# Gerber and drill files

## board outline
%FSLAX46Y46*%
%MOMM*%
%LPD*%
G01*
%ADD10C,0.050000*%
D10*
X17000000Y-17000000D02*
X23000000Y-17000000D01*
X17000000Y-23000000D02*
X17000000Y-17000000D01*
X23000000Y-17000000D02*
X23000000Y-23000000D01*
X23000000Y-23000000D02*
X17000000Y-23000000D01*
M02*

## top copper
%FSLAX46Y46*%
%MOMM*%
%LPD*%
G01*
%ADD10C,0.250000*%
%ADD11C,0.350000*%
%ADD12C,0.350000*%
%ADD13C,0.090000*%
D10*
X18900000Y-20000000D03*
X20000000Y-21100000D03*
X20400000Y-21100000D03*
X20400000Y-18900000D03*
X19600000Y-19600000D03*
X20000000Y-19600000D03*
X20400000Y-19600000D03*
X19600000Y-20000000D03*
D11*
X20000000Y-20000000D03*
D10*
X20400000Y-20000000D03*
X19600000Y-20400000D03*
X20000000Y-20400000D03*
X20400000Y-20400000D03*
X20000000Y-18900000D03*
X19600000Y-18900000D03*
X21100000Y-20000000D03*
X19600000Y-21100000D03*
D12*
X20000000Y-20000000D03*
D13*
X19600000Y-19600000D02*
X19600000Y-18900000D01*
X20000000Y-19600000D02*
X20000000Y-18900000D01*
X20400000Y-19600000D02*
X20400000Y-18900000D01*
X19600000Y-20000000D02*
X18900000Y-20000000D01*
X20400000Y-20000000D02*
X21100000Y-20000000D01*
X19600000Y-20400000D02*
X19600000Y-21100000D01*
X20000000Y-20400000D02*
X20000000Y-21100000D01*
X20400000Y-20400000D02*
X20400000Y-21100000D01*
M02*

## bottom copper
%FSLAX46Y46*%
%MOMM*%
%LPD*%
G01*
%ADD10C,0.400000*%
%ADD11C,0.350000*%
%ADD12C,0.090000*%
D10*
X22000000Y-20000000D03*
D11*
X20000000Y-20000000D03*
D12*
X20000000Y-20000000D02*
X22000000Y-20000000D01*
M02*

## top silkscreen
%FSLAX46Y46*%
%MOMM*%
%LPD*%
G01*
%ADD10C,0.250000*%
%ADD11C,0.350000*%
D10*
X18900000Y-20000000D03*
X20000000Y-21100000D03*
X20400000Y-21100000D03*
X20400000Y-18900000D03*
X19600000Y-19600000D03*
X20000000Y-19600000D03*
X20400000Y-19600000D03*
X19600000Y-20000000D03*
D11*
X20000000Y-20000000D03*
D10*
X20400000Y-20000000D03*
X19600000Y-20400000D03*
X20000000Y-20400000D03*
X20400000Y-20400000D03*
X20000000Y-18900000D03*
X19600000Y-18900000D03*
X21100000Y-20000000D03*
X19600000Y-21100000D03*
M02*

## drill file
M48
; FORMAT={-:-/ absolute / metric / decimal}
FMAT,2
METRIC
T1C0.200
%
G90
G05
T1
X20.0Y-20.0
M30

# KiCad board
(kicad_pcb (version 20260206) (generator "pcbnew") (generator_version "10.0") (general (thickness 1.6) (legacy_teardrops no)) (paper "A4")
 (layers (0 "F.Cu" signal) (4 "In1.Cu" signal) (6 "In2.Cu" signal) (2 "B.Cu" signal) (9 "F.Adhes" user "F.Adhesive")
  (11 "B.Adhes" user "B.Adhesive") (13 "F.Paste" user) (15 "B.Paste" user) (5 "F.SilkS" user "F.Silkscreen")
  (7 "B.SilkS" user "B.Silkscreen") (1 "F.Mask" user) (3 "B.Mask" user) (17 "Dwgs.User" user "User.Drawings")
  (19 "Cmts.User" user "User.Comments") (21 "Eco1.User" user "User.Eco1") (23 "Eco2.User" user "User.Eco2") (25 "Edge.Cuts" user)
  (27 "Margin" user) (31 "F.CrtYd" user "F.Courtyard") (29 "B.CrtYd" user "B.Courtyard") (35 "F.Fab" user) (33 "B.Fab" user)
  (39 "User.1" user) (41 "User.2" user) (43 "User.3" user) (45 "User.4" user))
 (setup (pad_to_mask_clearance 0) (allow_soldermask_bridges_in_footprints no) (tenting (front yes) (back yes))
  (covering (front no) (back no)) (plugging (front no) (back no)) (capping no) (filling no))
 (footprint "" (layer "F.Cu") (at 18.9 20)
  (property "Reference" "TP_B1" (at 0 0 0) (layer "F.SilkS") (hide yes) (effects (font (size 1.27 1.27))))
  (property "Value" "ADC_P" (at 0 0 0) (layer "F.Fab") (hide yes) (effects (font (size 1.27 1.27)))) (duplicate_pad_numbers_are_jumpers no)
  (pad "1" smd circle (at 0 0) (size 0.25 0.25) (layers "F.Cu" "F.Mask" "F.SilkS" "F.Adhes" "F.Paste" "F.CrtYd" "F.Fab") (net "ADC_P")))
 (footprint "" (layer "F.Cu") (at 20 21.1)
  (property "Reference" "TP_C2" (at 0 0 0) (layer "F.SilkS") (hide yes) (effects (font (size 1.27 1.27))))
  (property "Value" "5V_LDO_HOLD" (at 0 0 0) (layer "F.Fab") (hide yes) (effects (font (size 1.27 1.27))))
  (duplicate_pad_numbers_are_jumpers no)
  (pad "1" smd circle (at 0 0) (size 0.25 0.25)
   (layers "F.Cu" "F.Mask" "F.SilkS" "F.Adhes" "F.Paste" "F.CrtYd" "F.Fab") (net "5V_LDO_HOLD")))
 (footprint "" (layer "F.Cu") (at 22 20)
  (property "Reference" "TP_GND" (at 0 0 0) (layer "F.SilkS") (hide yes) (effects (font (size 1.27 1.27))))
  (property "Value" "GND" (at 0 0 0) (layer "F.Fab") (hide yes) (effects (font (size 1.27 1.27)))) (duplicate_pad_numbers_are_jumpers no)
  (pad "1" smd circle (at 0 0) (size 0.4 0.4) (layers "B.Cu" "B.Mask" "B.SilkS" "B.Adhes" "B.Paste" "B.CrtYd" "B.Fab") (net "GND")))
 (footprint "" (layer "F.Cu") (at 20.4 21.1)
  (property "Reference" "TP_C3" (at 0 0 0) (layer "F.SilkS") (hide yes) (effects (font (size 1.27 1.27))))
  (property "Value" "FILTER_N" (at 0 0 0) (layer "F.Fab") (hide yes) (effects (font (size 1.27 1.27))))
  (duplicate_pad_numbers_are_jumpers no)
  (pad "1" smd circle (at 0 0) (size 0.25 0.25) (layers "F.Cu" "F.Mask" "F.SilkS" "F.Adhes" "F.Paste" "F.CrtYd" "F.Fab") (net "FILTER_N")))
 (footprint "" (layer "F.Cu") (at 20.4 18.9)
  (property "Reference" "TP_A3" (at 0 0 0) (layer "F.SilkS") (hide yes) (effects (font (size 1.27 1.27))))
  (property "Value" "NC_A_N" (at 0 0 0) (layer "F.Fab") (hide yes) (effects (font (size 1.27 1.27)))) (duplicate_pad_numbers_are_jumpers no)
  (pad "1" smd circle (at 0 0) (size 0.25 0.25) (layers "F.Cu" "F.Mask" "F.SilkS" "F.Adhes" "F.Paste" "F.CrtYd" "F.Fab") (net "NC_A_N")))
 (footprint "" (layer "F.Cu") (at 20 20)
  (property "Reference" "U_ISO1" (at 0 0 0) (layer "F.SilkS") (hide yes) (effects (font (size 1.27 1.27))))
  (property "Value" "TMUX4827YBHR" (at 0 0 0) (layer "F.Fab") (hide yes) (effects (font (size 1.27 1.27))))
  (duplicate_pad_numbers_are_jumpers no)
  (pad "A1" smd circle (at -0.4 -0.4) (size 0.25 0.25)
   (layers "F.Cu" "F.Mask" "F.SilkS" "F.Adhes" "F.Paste" "F.CrtYd" "F.Fab") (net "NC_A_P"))
  (pad "A2" smd circle (at 0 -0.4) (size 0.25 0.25)
   (layers "F.Cu" "F.Mask" "F.SilkS" "F.Adhes" "F.Paste" "F.CrtYd" "F.Fab") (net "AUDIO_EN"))
  (pad "A3" smd circle (at 0.4 -0.4) (size 0.25 0.25)
   (layers "F.Cu" "F.Mask" "F.SilkS" "F.Adhes" "F.Paste" "F.CrtYd" "F.Fab") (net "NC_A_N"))
  (pad "B1" smd circle (at -0.4 0) (size 0.25 0.25) (layers "F.Cu" "F.Mask" "F.SilkS" "F.Adhes" "F.Paste" "F.CrtYd" "F.Fab") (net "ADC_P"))
  (pad "B2" smd circle (at 0 0) (size 0.35 0.35)
   (layers "F.Cu" "F.Mask" "F.SilkS" "F.Adhes" "F.Paste" "F.CrtYd" "F.Fab") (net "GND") (solder_mask_margin -0.05)
   (solder_paste_margin -0.05))
  (pad "B3" smd circle (at 0.4 0) (size 0.25 0.25) (layers "F.Cu" "F.Mask" "F.SilkS" "F.Adhes" "F.Paste" "F.CrtYd" "F.Fab") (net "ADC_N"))
  (pad "C1" smd circle (at -0.4 0.4) (size 0.25 0.25)
   (layers "F.Cu" "F.Mask" "F.SilkS" "F.Adhes" "F.Paste" "F.CrtYd" "F.Fab") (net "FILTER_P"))
  (pad "C2" smd circle (at 0 0.4) (size 0.25 0.25)
   (layers "F.Cu" "F.Mask" "F.SilkS" "F.Adhes" "F.Paste" "F.CrtYd" "F.Fab") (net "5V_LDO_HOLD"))
  (pad "C3" smd circle (at 0.4 0.4) (size 0.25 0.25)
   (layers "F.Cu" "F.Mask" "F.SilkS" "F.Adhes" "F.Paste" "F.CrtYd" "F.Fab") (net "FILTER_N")))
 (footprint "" (layer "F.Cu") (at 20 18.9)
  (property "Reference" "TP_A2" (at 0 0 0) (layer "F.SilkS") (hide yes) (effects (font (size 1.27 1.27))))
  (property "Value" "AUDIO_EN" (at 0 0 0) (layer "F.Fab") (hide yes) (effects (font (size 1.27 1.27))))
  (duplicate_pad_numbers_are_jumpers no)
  (pad "1" smd circle (at 0 0) (size 0.25 0.25) (layers "F.Cu" "F.Mask" "F.SilkS" "F.Adhes" "F.Paste" "F.CrtYd" "F.Fab") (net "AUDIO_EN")))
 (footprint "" (layer "F.Cu") (at 19.6 18.9)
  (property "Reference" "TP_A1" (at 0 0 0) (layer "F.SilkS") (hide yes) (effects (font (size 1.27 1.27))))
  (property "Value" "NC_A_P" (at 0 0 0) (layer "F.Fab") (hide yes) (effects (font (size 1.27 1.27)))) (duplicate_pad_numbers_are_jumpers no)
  (pad "1" smd circle (at 0 0) (size 0.25 0.25) (layers "F.Cu" "F.Mask" "F.SilkS" "F.Adhes" "F.Paste" "F.CrtYd" "F.Fab") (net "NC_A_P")))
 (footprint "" (layer "F.Cu") (at 21.1 20)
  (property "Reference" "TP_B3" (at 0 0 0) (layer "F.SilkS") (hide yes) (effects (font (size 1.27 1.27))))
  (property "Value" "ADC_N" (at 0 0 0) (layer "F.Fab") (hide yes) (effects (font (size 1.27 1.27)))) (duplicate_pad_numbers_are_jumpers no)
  (pad "1" smd circle (at 0 0) (size 0.25 0.25) (layers "F.Cu" "F.Mask" "F.SilkS" "F.Adhes" "F.Paste" "F.CrtYd" "F.Fab") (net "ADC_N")))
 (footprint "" (layer "F.Cu") (at 19.6 21.1)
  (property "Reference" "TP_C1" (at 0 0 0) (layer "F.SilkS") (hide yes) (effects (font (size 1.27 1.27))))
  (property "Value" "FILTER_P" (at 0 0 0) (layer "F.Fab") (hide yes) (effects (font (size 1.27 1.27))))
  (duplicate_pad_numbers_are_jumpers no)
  (pad "1" smd circle (at 0 0) (size 0.25 0.25) (layers "F.Cu" "F.Mask" "F.SilkS" "F.Adhes" "F.Paste" "F.CrtYd" "F.Fab") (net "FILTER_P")))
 (gr_line (start 17 17) (end 23 17) (stroke (width 0.05) (type default)) (layer "Edge.Cuts"))
 (gr_line (start 17 23) (end 17 17) (stroke (width 0.05) (type default)) (layer "Edge.Cuts"))
 (gr_line (start 23 17) (end 23 23) (stroke (width 0.05) (type default)) (layer "Edge.Cuts"))
 (gr_line (start 23 23) (end 17 23) (stroke (width 0.05) (type default)) (layer "Edge.Cuts"))
 (segment (start 19.6 19.6) (end 19.6 18.9) (width 0.09) (layer "F.Cu") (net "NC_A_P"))
 (segment (start 20 19.6) (end 20 18.9) (width 0.09) (layer "F.Cu") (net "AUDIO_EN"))
 (segment (start 20.4 19.6) (end 20.4 18.9) (width 0.09) (layer "F.Cu") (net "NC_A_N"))
 (segment (start 19.6 20) (end 18.9 20) (width 0.09) (layer "F.Cu") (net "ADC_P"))
 (via (at 20 20) (size 0.35) (drill 0.2) (layers "F.Cu" "B.Cu") (capping yes) (filling yes) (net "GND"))
 (segment (start 20 20) (end 22 20) (width 0.09) (layer "B.Cu") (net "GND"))
 (segment (start 20.4 20) (end 21.1 20) (width 0.09) (layer "F.Cu") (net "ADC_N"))
 (segment (start 19.6 20.4) (end 19.6 21.1) (width 0.09) (layer "F.Cu") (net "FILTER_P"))
 (segment (start 20 20.4) (end 20 21.1) (width 0.09) (layer "F.Cu") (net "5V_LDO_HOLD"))
 (segment (start 20.4 20.4) (end 20.4 21.1) (width 0.09) (layer "F.Cu") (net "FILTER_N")))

